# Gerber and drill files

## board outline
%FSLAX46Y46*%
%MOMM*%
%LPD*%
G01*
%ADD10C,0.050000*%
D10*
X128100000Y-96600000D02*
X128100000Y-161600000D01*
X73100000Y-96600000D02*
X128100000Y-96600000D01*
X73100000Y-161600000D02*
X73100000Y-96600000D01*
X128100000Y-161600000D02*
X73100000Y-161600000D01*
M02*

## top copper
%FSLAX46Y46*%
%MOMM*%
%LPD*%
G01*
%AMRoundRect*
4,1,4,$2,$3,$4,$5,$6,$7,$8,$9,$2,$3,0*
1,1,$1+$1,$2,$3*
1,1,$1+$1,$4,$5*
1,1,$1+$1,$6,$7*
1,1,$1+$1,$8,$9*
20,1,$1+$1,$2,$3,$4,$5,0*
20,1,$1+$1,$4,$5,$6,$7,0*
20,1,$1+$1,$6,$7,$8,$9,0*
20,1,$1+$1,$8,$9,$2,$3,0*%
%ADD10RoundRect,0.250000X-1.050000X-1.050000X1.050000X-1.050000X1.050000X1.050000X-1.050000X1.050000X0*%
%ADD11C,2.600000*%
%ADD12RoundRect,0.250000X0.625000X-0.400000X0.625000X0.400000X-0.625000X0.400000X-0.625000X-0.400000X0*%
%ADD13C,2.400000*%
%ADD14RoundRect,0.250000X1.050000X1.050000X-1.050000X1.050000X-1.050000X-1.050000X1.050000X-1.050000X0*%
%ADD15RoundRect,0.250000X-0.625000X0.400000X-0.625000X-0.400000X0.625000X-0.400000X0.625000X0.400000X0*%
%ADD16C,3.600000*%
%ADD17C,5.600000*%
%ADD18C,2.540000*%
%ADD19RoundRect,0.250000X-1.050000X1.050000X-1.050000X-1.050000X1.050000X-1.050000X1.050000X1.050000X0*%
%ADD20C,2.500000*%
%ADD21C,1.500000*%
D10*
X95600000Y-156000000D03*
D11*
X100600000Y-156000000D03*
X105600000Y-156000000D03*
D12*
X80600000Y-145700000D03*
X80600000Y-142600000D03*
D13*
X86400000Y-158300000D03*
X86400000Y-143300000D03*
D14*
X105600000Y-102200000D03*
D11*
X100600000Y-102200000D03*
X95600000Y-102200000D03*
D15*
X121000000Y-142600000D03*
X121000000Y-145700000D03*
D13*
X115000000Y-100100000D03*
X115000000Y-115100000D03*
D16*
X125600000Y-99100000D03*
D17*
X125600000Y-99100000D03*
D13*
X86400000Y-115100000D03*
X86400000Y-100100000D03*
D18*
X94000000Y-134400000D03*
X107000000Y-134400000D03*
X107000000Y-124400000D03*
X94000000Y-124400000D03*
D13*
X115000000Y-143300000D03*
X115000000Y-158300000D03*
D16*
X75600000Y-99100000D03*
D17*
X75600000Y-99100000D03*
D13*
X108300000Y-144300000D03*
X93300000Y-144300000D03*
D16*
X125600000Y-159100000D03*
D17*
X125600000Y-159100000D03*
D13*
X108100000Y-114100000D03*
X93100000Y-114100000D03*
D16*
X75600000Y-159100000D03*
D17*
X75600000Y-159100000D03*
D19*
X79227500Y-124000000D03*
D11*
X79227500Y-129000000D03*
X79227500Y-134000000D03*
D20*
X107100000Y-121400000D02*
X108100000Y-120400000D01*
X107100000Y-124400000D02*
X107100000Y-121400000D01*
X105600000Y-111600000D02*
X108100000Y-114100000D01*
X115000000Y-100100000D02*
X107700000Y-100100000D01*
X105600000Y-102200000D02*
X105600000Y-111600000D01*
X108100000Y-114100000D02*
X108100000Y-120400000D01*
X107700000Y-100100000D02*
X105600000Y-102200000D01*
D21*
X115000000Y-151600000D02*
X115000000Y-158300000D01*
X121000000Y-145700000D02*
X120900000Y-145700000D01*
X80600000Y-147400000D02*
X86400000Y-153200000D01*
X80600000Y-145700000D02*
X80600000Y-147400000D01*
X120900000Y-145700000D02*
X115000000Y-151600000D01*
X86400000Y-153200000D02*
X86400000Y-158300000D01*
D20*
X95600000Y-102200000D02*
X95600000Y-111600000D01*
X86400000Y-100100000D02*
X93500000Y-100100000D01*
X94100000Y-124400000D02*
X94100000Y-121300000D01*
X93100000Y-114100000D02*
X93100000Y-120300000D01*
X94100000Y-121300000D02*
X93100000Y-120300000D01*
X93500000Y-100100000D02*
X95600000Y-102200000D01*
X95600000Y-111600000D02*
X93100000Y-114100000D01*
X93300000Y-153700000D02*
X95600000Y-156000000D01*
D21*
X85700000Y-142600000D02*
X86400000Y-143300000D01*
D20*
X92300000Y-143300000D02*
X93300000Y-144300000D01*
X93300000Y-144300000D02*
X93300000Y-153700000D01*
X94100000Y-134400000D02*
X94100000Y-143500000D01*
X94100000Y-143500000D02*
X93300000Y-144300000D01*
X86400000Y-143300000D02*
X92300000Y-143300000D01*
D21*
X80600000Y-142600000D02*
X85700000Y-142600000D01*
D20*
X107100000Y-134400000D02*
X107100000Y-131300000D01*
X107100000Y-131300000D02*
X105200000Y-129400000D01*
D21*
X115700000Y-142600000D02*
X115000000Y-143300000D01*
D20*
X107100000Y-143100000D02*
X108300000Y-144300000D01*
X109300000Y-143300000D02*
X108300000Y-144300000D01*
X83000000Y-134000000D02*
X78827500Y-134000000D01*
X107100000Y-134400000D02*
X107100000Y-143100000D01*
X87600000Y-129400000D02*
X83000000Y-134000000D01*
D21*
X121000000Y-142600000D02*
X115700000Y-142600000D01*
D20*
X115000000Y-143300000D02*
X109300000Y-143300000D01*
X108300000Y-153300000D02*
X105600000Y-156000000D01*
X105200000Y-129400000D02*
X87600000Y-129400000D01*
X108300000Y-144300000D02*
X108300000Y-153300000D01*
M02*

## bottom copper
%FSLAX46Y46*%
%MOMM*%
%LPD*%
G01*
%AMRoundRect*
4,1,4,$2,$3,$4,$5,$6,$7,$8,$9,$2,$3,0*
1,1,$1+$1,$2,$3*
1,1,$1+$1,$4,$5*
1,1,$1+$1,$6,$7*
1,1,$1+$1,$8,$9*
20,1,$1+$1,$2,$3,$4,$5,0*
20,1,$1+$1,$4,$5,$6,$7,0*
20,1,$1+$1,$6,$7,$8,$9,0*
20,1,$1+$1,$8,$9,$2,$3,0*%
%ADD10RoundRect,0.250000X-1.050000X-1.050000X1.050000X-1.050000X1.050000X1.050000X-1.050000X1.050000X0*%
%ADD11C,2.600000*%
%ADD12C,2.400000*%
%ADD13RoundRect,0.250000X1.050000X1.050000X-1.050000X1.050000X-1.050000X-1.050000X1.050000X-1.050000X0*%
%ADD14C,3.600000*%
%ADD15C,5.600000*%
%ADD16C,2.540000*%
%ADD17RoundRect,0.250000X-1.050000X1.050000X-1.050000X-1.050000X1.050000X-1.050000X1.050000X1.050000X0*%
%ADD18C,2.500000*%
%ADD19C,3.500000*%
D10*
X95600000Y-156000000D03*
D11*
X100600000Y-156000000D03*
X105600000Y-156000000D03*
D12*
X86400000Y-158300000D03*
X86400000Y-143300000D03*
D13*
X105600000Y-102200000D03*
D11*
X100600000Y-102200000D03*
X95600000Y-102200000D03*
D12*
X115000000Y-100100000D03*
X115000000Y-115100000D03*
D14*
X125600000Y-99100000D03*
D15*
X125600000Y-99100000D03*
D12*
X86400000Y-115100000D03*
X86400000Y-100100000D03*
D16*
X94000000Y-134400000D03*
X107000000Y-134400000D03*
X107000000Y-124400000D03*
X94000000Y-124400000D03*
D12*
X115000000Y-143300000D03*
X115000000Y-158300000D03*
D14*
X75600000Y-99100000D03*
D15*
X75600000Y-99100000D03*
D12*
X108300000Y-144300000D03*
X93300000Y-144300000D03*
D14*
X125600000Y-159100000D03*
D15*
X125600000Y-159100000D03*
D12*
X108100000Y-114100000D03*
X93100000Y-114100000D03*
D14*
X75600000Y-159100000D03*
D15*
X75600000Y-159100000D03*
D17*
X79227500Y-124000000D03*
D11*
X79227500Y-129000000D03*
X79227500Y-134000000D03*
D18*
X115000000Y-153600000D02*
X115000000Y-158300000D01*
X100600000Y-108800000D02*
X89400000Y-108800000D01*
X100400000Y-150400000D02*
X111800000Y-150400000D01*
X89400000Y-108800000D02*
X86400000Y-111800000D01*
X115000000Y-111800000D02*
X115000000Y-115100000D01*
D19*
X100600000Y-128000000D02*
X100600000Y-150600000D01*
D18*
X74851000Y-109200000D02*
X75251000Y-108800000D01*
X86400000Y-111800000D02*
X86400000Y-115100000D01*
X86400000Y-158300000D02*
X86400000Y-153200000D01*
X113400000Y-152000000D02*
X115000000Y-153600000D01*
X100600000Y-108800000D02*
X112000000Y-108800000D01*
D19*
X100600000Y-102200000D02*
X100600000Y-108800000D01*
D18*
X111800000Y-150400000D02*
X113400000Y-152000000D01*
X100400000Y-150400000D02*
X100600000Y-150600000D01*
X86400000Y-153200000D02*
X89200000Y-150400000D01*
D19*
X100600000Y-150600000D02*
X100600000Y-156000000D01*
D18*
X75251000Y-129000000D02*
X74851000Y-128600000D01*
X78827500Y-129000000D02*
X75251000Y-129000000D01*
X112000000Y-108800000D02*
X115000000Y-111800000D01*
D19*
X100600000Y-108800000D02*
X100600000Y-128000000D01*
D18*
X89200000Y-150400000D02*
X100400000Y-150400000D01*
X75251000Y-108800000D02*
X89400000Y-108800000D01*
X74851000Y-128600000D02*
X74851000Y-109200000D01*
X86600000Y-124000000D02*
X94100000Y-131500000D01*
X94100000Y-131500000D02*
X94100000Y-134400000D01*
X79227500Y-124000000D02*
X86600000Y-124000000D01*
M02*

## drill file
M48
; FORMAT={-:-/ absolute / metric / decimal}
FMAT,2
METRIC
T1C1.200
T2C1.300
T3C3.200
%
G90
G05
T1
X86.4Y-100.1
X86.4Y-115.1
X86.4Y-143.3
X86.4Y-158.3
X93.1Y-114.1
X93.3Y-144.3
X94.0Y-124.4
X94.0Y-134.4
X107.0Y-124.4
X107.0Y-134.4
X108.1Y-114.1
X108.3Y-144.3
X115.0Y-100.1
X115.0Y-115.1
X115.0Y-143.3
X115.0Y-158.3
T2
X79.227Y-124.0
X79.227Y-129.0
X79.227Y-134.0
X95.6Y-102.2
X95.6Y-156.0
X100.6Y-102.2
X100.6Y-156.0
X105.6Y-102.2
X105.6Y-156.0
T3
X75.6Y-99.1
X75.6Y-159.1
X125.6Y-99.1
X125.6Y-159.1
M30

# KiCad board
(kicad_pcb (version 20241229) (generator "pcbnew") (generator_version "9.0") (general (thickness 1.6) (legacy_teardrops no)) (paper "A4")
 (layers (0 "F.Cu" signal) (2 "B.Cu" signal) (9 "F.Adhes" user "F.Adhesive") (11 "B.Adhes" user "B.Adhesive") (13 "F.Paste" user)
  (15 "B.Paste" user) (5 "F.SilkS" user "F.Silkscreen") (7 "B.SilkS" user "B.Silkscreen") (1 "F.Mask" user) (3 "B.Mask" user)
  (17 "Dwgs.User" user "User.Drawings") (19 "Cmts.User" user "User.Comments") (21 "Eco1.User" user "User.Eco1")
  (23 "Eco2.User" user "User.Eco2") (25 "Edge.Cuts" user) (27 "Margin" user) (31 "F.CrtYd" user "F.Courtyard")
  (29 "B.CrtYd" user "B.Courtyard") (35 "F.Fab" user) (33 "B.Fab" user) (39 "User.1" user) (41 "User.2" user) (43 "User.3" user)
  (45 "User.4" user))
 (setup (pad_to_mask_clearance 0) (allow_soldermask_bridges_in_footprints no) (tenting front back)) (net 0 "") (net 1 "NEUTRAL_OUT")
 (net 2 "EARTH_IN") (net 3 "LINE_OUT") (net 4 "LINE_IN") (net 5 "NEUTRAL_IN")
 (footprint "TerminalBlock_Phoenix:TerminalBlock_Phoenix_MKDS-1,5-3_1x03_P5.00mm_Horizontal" (layer "F.Cu") (at 95.6 156)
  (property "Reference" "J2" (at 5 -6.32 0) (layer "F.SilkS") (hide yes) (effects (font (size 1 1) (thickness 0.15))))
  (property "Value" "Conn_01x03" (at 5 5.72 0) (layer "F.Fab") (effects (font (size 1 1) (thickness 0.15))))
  (pad "1" thru_hole roundrect (at 0 0) (size 2.6 2.6) (drill 1.3) (layers "*.Cu" "*.Mask") (remove_unused_layers no)
   (roundrect_rratio 0.096154) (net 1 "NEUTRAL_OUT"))
  (pad "2" thru_hole circle (at 5 0) (size 2.6 2.6) (drill 1.3) (layers "*.Cu" "*.Mask") (remove_unused_layers no) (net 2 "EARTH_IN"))
  (pad "3" thru_hole circle (at 10 0) (size 2.6 2.6) (drill 1.3) (layers "*.Cu" "*.Mask") (remove_unused_layers no) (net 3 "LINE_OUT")))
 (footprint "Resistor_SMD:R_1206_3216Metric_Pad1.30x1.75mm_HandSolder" (layer "F.Cu") (at 80.6 144.15 90)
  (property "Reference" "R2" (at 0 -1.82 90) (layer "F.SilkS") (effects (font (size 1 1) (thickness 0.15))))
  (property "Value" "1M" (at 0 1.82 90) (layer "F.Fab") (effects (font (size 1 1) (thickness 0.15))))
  (pad "1" smd roundrect (at -1.55 0 90) (size 1.3 1.75) (layers "F.Cu" "F.Mask" "F.Paste") (roundrect_rratio 0.192308) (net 2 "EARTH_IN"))
  (pad "2" smd roundrect (at 1.55 0 90) (size 1.3 1.75) (layers "F.Cu" "F.Mask" "F.Paste") (roundrect_rratio 0.192308) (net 1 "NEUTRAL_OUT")))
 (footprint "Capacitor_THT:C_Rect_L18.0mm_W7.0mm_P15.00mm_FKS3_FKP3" (layer "F.Cu") (at 86.4 158.3 90)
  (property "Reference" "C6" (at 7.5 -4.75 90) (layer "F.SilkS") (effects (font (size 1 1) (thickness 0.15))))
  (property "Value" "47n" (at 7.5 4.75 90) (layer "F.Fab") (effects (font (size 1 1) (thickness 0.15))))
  (pad "1" thru_hole circle (at 0 0 90) (size 2.4 2.4) (drill 1.2) (layers "*.Cu" "*.Mask") (remove_unused_layers no) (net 2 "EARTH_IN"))
  (pad "2" thru_hole circle (at 15 0 90) (size 2.4 2.4) (drill 1.2) (layers "*.Cu" "*.Mask") (remove_unused_layers no) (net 1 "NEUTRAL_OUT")))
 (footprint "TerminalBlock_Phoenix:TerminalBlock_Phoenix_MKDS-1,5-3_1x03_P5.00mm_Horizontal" (layer "F.Cu") (at 105.6 102.2 180)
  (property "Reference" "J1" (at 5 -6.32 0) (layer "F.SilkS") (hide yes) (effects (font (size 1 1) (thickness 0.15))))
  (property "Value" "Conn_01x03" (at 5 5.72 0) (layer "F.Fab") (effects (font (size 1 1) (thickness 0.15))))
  (pad "1" thru_hole roundrect (at 0 0 180) (size 2.6 2.6) (drill 1.3) (layers "*.Cu" "*.Mask") (remove_unused_layers no)
   (roundrect_rratio 0.096154) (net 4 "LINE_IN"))
  (pad "2" thru_hole circle (at 5 0 180) (size 2.6 2.6) (drill 1.3) (layers "*.Cu" "*.Mask") (remove_unused_layers no) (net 2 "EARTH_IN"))
  (pad "3" thru_hole circle (at 10 0 180) (size 2.6 2.6) (drill 1.3) (layers "*.Cu" "*.Mask") (remove_unused_layers no) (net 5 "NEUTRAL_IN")))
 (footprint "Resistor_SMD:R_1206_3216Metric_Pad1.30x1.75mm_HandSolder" (layer "F.Cu") (at 121 144.15 -90)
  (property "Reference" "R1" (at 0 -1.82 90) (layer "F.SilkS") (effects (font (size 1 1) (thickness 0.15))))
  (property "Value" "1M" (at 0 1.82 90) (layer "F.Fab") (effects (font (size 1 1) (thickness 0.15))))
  (pad "1" smd roundrect (at -1.55 0 270) (size 1.3 1.75) (layers "F.Cu" "F.Mask" "F.Paste") (roundrect_rratio 0.192308) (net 3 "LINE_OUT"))
  (pad "2" smd roundrect (at 1.55 0 270) (size 1.3 1.75) (layers "F.Cu" "F.Mask" "F.Paste") (roundrect_rratio 0.192308) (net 2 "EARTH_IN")))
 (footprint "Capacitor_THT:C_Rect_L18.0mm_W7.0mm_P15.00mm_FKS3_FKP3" (layer "F.Cu") (at 115 100.1 -90)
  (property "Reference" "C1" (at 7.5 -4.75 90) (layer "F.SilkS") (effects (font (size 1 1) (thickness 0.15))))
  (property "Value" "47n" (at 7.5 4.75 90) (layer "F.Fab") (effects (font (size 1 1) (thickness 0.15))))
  (pad "1" thru_hole circle (at 0 0 270) (size 2.4 2.4) (drill 1.2) (layers "*.Cu" "*.Mask") (remove_unused_layers no) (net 4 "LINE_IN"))
  (pad "2" thru_hole circle (at 15 0 270) (size 2.4 2.4) (drill 1.2) (layers "*.Cu" "*.Mask") (remove_unused_layers no) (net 2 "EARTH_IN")))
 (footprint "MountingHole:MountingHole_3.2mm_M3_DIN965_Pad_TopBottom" (layer "F.Cu") (at 125.6 99.1)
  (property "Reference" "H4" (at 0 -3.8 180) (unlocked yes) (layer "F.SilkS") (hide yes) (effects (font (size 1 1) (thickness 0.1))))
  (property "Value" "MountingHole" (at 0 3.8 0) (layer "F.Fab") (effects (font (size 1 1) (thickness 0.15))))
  (pad "1" thru_hole circle (at 0 0) (size 3.6 3.6) (drill 3.2) (layers "*.Cu" "*.Mask") (remove_unused_layers no))
  (pad "1" connect circle (at 0 0) (size 5.6 5.6) (layers "F.Cu" "F.Mask"))
  (pad "1" connect circle (at 0 0) (size 5.6 5.6) (layers "B.Cu" "B.Mask")))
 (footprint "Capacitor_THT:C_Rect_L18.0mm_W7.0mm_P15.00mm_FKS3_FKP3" (layer "F.Cu") (at 86.4 115.1 90)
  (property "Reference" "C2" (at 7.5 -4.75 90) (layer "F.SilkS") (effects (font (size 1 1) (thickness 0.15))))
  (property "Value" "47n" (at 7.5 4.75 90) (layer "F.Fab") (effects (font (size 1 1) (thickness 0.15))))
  (pad "1" thru_hole circle (at 0 0 90) (size 2.4 2.4) (drill 1.2) (layers "*.Cu" "*.Mask") (remove_unused_layers no) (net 2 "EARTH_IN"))
  (pad "2" thru_hole circle (at 15 0 90) (size 2.4 2.4) (drill 1.2) (layers "*.Cu" "*.Mask") (remove_unused_layers no) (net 5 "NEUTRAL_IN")))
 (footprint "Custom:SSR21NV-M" (layer "F.Cu") (at 100.5 129.4)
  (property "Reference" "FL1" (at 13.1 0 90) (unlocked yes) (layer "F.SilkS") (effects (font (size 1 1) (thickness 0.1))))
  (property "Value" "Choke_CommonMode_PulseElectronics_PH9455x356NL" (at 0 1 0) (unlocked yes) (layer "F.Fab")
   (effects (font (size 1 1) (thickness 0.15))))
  (pad "1" thru_hole circle (at -6.5 5) (size 2.54 2.54) (drill 1.2) (layers "*.Cu" "*.Mask") (remove_unused_layers no)
   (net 1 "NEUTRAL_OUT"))
  (pad "2" thru_hole circle (at 6.5 5) (size 2.54 2.54) (drill 1.2) (layers "*.Cu" "*.Mask") (remove_unused_layers no) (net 3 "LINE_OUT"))
  (pad "3" thru_hole circle (at 6.5 -5) (size 2.54 2.54) (drill 1.2) (layers "*.Cu" "*.Mask") (remove_unused_layers no) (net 4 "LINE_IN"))
  (pad "4" thru_hole circle (at -6.5 -5) (size 2.54 2.54) (drill 1.2) (layers "*.Cu" "*.Mask") (remove_unused_layers no)
   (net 5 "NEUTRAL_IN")))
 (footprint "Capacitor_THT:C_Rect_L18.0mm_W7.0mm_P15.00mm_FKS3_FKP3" (layer "F.Cu") (at 115 143.3 -90)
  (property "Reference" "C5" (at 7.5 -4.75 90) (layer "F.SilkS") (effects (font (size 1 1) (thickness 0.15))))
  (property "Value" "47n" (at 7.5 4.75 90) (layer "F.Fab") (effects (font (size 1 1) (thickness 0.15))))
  (pad "1" thru_hole circle (at 0 0 270) (size 2.4 2.4) (drill 1.2) (layers "*.Cu" "*.Mask") (remove_unused_layers no) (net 3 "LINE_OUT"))
  (pad "2" thru_hole circle (at 15 0 270) (size 2.4 2.4) (drill 1.2) (layers "*.Cu" "*.Mask") (remove_unused_layers no) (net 2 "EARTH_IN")))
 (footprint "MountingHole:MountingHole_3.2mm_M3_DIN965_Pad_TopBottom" (layer "F.Cu") (at 75.6 99.1)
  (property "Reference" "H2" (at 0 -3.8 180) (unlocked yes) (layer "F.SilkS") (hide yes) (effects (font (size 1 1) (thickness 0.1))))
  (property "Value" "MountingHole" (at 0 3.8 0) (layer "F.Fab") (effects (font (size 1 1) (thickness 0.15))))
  (pad "1" thru_hole circle (at 0 0) (size 3.6 3.6) (drill 3.2) (layers "*.Cu" "*.Mask") (remove_unused_layers no))
  (pad "1" connect circle (at 0 0) (size 5.6 5.6) (layers "F.Cu" "F.Mask"))
  (pad "1" connect circle (at 0 0) (size 5.6 5.6) (layers "B.Cu" "B.Mask")))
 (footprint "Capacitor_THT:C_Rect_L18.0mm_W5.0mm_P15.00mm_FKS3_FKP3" (layer "F.Cu") (at 108.3 144.3 180)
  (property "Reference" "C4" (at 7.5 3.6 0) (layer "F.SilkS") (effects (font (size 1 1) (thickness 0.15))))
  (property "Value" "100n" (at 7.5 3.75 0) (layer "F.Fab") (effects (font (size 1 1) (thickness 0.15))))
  (pad "1" thru_hole circle (at 0 0 180) (size 2.4 2.4) (drill 1.2) (layers "*.Cu" "*.Mask") (remove_unused_layers no) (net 3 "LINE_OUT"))
  (pad "2" thru_hole circle (at 15 0 180) (size 2.4 2.4) (drill 1.2) (layers "*.Cu" "*.Mask") (remove_unused_layers no)
   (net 1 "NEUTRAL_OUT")))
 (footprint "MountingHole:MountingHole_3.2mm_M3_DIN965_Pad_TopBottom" (layer "F.Cu") (at 125.6 159.1)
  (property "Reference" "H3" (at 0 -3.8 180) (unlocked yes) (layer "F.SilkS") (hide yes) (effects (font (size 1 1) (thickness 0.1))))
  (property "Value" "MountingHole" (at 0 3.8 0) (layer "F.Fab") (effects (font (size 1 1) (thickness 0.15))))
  (pad "1" thru_hole circle (at 0 0) (size 3.6 3.6) (drill 3.2) (layers "*.Cu" "*.Mask") (remove_unused_layers no))
  (pad "1" connect circle (at 0 0) (size 5.6 5.6) (layers "F.Cu" "F.Mask"))
  (pad "1" connect circle (at 0 0) (size 5.6 5.6) (layers "B.Cu" "B.Mask")))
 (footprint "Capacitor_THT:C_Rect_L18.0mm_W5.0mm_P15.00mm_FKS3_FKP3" (layer "F.Cu") (at 108.1 114.1 180)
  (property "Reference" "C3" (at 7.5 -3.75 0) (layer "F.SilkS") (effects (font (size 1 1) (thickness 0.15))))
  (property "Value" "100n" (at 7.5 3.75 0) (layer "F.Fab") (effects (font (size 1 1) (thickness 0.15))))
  (pad "1" thru_hole circle (at 0 0 180) (size 2.4 2.4) (drill 1.2) (layers "*.Cu" "*.Mask") (remove_unused_layers no) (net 4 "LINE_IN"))
  (pad "2" thru_hole circle (at 15 0 180) (size 2.4 2.4) (drill 1.2) (layers "*.Cu" "*.Mask") (remove_unused_layers no) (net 5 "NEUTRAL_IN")))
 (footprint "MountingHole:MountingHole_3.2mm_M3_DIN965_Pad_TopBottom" (layer "F.Cu") (at 75.6 159.1)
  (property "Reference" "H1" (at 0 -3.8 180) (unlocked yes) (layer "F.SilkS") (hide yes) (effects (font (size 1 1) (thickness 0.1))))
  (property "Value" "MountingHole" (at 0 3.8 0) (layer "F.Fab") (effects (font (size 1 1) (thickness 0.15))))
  (pad "1" thru_hole circle (at 0 0) (size 3.6 3.6) (drill 3.2) (layers "*.Cu" "*.Mask") (remove_unused_layers no))
  (pad "1" connect circle (at 0 0) (size 5.6 5.6) (layers "F.Cu" "F.Mask"))
  (pad "1" connect circle (at 0 0) (size 5.6 5.6) (layers "B.Cu" "B.Mask")))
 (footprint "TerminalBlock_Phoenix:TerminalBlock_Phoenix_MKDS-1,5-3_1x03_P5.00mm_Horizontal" (layer "F.Cu") (at 79.2275 124 -90)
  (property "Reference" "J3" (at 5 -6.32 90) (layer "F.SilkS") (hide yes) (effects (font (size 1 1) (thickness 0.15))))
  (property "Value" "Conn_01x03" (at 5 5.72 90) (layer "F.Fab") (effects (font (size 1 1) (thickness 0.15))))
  (pad "1" thru_hole roundrect (at 0 0 270) (size 2.6 2.6) (drill 1.3) (layers "*.Cu" "*.Mask") (remove_unused_layers no)
   (roundrect_rratio 0.096154) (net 1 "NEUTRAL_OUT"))
  (pad "2" thru_hole circle (at 5 0 270) (size 2.6 2.6) (drill 1.3) (layers "*.Cu" "*.Mask") (remove_unused_layers no) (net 2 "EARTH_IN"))
  (pad "3" thru_hole circle (at 10 0 270) (size 2.6 2.6) (drill 1.3) (layers "*.Cu" "*.Mask") (remove_unused_layers no) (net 3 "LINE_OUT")))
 (gr_line (start 128.1 96.6) (end 128.1 161.6) (stroke (width 0.05) (type default)) (layer "Edge.Cuts"))
 (gr_line (start 73.1 96.6) (end 128.1 96.6) (stroke (width 0.05) (type default)) (layer "Edge.Cuts"))
 (gr_line (start 73.1 161.6) (end 73.1 96.6) (stroke (width 0.05) (type default)) (layer "Edge.Cuts"))
 (gr_line (start 128.1 161.6) (end 73.1 161.6) (stroke (width 0.05) (type default)) (layer "Edge.Cuts"))
 (segment (start 107.1 121.4) (end 108.1 120.4) (width 2.5) (layer "F.Cu") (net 4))
 (segment (start 107.1 124.4) (end 107.1 121.4) (width 2.5) (layer "F.Cu") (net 4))
 (segment (start 105.6 111.6) (end 108.1 114.1) (width 2.5) (layer "F.Cu") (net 4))
 (segment (start 115 100.1) (end 107.7 100.1) (width 2.5) (layer "F.Cu") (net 4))
 (segment (start 105.6 102.2) (end 105.6 111.6) (width 2.5) (layer "F.Cu") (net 4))
 (segment (start 108.1 114.1) (end 108.1 120.4) (width 2.5) (layer "F.Cu") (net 4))
 (segment (start 107.7 100.1) (end 105.6 102.2) (width 2.5) (layer "F.Cu") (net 4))
 (segment (start 115 151.6) (end 115 158.3) (width 1.5) (layer "F.Cu") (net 2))
 (segment (start 121 145.7) (end 120.9 145.7) (width 1.5) (layer "F.Cu") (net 2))
 (segment (start 80.6 147.4) (end 86.4 153.2) (width 1.5) (layer "F.Cu") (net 2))
 (segment (start 80.6 145.7) (end 80.6 147.4) (width 1.5) (layer "F.Cu") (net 2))
 (segment (start 120.9 145.7) (end 115 151.6) (width 1.5) (layer "F.Cu") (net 2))
 (segment (start 86.4 153.2) (end 86.4 158.3) (width 1.5) (layer "F.Cu") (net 2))
 (segment (start 115 153.6) (end 115 158.3) (width 2.5) (layer "B.Cu") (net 2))
 (segment (start 100.6 108.8) (end 89.4 108.8) (width 2.5) (layer "B.Cu") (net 2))
 (segment (start 100.4 150.4) (end 111.8 150.4) (width 2.5) (layer "B.Cu") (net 2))
 (segment (start 89.4 108.8) (end 86.4 111.8) (width 2.5) (layer "B.Cu") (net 2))
 (segment (start 115 111.8) (end 115 115.1) (width 2.5) (layer "B.Cu") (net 2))
 (segment (start 100.6 128) (end 100.6 150.6) (width 3.5) (layer "B.Cu") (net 2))
 (segment (start 74.851 109.2) (end 75.251 108.8) (width 2.5) (layer "B.Cu") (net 2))
 (segment (start 86.4 111.8) (end 86.4 115.1) (width 2.5) (layer "B.Cu") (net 2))
 (segment (start 86.4 158.3) (end 86.4 153.2) (width 2.5) (layer "B.Cu") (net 2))
 (segment (start 113.4 152) (end 115 153.6) (width 2.5) (layer "B.Cu") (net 2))
 (segment (start 100.6 108.8) (end 112 108.8) (width 2.5) (layer "B.Cu") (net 2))
 (segment (start 100.6 102.2) (end 100.6 108.8) (width 3.5) (layer "B.Cu") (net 2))
 (segment (start 111.8 150.4) (end 113.4 152) (width 2.5) (layer "B.Cu") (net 2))
 (segment (start 100.4 150.4) (end 100.6 150.6) (width 2.5) (layer "B.Cu") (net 2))
 (segment (start 86.4 153.2) (end 89.2 150.4) (width 2.5) (layer "B.Cu") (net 2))
 (segment (start 100.6 150.6) (end 100.6 156) (width 3.5) (layer "B.Cu") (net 2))
 (segment (start 75.251 129) (end 74.851 128.6) (width 2.5) (layer "B.Cu") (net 2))
 (segment (start 78.8275 129) (end 75.251 129) (width 2.5) (layer "B.Cu") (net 2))
 (segment (start 112 108.8) (end 115 111.8) (width 2.5) (layer "B.Cu") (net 2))
 (segment (start 100.6 108.8) (end 100.6 128) (width 3.5) (layer "B.Cu") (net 2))
 (segment (start 89.2 150.4) (end 100.4 150.4) (width 2.5) (layer "B.Cu") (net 2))
 (segment (start 75.251 108.8) (end 89.4 108.8) (width 2.5) (layer "B.Cu") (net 2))
 (segment (start 74.851 128.6) (end 74.851 109.2) (width 2.5) (layer "B.Cu") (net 2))
 (segment (start 95.6 102.2) (end 95.6 111.6) (width 2.5) (layer "F.Cu") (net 5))
 (segment (start 86.4 100.1) (end 93.5 100.1) (width 2.5) (layer "F.Cu") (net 5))
 (segment (start 94.1 124.4) (end 94.1 121.3) (width 2.5) (layer "F.Cu") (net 5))
 (segment (start 93.1 114.1) (end 93.1 120.3) (width 2.5) (layer "F.Cu") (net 5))
 (segment (start 94.1 121.3) (end 93.1 120.3) (width 2.5) (layer "F.Cu") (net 5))
 (segment (start 93.5 100.1) (end 95.6 102.2) (width 2.5) (layer "F.Cu") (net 5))
 (segment (start 95.6 111.6) (end 93.1 114.1) (width 2.5) (layer "F.Cu") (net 5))
 (segment (start 93.3 153.7) (end 95.6 156) (width 2.5) (layer "F.Cu") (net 1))
 (segment (start 85.7 142.6) (end 86.4 143.3) (width 1.5) (layer "F.Cu") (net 1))
 (segment (start 92.3 143.3) (end 93.3 144.3) (width 2.5) (layer "F.Cu") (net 1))
 (segment (start 93.3 144.3) (end 93.3 153.7) (width 2.5) (layer "F.Cu") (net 1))
 (segment (start 94.1 134.4) (end 94.1 143.5) (width 2.5) (layer "F.Cu") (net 1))
 (segment (start 94.1 143.5) (end 93.3 144.3) (width 2.5) (layer "F.Cu") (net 1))
 (segment (start 86.4 143.3) (end 92.3 143.3) (width 2.5) (layer "F.Cu") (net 1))
 (segment (start 80.6 142.6) (end 85.7 142.6) (width 1.5) (layer "F.Cu") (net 1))
 (segment (start 86.6 124) (end 94.1 131.5) (width 2.5) (layer "B.Cu") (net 1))
 (segment (start 94.1 131.5) (end 94.1 134.4) (width 2.5) (layer "B.Cu") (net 1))
 (segment (start 79.2275 124) (end 86.6 124) (width 2.5) (layer "B.Cu") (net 1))
 (segment (start 107.1 134.4) (end 107.1 131.3) (width 2.5) (layer "F.Cu") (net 3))
 (segment (start 107.1 131.3) (end 105.2 129.4) (width 2.5) (layer "F.Cu") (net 3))
 (segment (start 115.7 142.6) (end 115 143.3) (width 1.5) (layer "F.Cu") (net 3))
 (segment (start 107.1 143.1) (end 108.3 144.3) (width 2.5) (layer "F.Cu") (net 3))
 (segment (start 109.3 143.3) (end 108.3 144.3) (width 2.5) (layer "F.Cu") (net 3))
 (segment (start 83 134) (end 78.8275 134) (width 2.5) (layer "F.Cu") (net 3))
 (segment (start 107.1 134.4) (end 107.1 143.1) (width 2.5) (layer "F.Cu") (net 3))
 (segment (start 87.6 129.4) (end 83 134) (width 2.5) (layer "F.Cu") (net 3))
 (segment (start 121 142.6) (end 115.7 142.6) (width 1.5) (layer "F.Cu") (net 3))
 (segment (start 115 143.3) (end 109.3 143.3) (width 2.5) (layer "F.Cu") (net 3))
 (segment (start 108.3 153.3) (end 105.6 156) (width 2.5) (layer "F.Cu") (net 3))
 (segment (start 105.2 129.4) (end 87.6 129.4) (width 2.5) (layer "F.Cu") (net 3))
 (segment (start 108.3 144.3) (end 108.3 153.3) (width 2.5) (layer "F.Cu") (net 3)))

